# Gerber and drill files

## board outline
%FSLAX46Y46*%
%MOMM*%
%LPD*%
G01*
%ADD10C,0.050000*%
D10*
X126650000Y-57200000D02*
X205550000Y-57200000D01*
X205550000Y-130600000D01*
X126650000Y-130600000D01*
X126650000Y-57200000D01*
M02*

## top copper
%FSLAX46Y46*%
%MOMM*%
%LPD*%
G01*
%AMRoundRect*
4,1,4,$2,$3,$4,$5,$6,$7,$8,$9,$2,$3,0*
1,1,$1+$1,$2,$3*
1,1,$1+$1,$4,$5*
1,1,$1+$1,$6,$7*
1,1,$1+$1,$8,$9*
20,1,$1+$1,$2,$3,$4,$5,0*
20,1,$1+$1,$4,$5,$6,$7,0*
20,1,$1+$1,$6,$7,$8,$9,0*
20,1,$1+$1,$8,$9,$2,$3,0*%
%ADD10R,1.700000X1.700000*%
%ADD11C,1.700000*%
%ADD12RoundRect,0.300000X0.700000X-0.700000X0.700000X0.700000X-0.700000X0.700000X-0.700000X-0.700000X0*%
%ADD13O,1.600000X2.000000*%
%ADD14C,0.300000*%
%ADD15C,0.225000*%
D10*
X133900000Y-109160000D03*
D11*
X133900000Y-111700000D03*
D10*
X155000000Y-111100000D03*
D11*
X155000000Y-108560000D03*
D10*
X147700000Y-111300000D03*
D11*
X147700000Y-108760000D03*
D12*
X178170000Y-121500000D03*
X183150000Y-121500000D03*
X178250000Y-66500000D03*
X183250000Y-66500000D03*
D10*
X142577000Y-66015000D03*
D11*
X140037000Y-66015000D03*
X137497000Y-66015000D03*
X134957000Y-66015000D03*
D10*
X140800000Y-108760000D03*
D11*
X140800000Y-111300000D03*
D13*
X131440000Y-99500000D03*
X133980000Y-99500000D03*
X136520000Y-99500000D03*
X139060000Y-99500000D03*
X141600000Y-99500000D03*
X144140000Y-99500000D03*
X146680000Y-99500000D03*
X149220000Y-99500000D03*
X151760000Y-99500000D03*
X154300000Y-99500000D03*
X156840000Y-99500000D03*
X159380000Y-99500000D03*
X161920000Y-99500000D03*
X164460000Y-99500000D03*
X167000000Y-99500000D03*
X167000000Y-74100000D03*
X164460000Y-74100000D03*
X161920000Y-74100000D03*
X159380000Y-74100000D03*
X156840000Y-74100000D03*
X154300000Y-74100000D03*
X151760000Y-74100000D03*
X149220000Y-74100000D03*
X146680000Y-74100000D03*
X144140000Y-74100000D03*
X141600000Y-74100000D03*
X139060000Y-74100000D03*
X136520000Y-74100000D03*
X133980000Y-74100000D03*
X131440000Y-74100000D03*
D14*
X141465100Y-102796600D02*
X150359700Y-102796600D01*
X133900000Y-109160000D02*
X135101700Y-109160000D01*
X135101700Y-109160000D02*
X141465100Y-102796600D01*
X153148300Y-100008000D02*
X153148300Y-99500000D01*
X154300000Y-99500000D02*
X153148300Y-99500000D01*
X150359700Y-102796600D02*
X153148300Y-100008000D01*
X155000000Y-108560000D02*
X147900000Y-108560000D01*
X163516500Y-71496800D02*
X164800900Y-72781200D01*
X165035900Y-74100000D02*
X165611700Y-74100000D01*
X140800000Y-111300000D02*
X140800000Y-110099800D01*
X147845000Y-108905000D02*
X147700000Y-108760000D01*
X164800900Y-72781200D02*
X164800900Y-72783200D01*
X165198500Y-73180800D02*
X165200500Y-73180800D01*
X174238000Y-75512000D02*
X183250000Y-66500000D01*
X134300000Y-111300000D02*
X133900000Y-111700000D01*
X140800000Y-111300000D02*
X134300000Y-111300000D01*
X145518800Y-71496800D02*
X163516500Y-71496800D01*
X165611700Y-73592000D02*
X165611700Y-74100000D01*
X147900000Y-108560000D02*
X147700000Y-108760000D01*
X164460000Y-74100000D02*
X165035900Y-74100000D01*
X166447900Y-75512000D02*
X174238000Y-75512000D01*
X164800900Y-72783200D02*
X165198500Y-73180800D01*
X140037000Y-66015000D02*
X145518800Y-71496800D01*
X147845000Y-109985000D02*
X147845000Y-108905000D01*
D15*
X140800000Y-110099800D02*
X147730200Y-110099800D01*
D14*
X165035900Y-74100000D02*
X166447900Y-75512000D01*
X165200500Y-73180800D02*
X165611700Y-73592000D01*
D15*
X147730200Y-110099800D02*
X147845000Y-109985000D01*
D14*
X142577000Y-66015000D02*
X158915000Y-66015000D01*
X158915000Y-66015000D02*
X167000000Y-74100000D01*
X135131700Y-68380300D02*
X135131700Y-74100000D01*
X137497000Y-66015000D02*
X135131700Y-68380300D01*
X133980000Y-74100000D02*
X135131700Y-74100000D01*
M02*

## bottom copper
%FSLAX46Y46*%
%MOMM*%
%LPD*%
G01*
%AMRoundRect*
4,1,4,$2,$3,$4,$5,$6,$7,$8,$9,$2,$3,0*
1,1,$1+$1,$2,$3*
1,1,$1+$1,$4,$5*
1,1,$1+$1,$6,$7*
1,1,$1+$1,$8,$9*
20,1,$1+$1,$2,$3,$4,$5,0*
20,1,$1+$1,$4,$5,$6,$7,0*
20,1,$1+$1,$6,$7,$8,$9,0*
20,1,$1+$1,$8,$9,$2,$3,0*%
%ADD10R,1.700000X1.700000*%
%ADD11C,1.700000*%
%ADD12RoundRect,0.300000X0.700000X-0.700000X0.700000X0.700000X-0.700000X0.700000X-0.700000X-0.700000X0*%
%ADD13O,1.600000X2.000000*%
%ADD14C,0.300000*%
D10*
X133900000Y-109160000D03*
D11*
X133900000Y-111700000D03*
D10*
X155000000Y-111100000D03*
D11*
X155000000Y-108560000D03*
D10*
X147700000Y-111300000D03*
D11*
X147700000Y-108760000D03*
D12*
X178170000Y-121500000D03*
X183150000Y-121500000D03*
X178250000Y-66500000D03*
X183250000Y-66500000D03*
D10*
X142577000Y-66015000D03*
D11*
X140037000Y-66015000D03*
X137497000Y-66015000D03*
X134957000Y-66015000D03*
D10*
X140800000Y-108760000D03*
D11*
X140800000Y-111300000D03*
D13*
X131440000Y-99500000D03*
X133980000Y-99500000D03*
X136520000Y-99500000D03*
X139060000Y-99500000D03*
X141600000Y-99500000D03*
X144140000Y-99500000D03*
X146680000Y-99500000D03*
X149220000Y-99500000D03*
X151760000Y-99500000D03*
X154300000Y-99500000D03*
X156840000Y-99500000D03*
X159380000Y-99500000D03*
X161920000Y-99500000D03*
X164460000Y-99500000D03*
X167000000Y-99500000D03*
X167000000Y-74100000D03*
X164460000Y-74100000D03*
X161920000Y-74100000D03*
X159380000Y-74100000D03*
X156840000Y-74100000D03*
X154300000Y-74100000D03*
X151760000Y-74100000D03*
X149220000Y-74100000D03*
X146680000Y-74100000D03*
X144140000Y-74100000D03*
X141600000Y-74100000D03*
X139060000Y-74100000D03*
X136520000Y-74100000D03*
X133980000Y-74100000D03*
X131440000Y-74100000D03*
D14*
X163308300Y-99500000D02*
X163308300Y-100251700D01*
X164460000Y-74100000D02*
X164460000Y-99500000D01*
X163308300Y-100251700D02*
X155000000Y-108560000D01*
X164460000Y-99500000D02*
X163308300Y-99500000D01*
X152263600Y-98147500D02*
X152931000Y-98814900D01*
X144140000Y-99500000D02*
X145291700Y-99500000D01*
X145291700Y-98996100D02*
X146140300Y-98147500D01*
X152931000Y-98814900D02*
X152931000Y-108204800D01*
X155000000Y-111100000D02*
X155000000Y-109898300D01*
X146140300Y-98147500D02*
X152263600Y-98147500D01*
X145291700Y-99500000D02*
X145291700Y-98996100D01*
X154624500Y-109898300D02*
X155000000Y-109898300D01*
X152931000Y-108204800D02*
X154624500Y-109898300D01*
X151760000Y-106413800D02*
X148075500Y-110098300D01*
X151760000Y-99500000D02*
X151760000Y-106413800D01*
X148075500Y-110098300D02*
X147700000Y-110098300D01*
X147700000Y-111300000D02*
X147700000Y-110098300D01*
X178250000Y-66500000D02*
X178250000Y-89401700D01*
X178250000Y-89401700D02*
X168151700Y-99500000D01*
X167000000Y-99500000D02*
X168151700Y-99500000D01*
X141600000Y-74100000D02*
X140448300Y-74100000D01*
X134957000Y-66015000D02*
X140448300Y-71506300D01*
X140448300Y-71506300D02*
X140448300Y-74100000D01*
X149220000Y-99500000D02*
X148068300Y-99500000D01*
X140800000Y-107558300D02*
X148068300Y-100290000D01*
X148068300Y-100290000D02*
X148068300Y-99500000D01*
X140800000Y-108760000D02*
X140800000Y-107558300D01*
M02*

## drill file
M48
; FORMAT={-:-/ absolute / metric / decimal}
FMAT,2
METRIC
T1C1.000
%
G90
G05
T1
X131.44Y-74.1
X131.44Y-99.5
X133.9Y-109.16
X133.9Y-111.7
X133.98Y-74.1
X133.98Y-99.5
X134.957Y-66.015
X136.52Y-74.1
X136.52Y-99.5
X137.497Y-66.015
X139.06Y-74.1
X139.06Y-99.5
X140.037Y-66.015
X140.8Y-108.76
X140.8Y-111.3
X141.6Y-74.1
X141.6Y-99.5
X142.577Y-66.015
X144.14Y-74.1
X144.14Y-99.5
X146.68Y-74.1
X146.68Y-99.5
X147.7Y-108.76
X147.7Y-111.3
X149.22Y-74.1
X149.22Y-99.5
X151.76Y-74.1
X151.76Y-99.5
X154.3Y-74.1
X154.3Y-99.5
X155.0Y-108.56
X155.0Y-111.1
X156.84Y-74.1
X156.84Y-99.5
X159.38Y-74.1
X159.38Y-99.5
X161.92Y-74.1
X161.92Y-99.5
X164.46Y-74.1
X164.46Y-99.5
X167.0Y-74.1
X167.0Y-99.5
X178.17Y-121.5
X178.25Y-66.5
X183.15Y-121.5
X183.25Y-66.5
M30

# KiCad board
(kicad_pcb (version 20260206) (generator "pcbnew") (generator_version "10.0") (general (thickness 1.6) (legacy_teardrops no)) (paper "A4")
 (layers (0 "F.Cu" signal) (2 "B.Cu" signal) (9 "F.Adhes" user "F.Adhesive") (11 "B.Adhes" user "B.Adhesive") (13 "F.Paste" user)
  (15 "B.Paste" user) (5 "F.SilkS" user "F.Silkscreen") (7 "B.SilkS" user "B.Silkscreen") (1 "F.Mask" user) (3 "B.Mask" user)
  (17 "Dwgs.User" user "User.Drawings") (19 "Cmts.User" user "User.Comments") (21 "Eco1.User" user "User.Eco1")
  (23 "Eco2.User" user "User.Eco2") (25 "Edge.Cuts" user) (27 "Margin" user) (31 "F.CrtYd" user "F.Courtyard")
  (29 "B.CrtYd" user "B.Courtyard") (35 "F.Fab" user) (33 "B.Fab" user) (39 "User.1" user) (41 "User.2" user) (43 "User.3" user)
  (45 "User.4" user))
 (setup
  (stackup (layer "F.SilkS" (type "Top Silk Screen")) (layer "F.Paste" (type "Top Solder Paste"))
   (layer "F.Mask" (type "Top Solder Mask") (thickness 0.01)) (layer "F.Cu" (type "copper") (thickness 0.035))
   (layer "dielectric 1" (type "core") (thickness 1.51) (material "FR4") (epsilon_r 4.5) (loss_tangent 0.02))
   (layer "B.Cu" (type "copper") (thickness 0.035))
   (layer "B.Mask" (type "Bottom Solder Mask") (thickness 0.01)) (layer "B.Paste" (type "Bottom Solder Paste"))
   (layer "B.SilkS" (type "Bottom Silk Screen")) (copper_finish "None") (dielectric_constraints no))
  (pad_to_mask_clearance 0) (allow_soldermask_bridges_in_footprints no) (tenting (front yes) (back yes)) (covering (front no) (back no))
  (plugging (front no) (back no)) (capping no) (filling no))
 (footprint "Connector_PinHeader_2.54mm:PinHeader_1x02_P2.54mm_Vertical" (layer "F.Cu") (at 133.9 109.16)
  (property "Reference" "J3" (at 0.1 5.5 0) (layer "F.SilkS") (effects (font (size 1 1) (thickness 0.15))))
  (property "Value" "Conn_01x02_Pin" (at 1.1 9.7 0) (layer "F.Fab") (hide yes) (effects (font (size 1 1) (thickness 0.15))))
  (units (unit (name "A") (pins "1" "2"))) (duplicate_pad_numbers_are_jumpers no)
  (pad "1" thru_hole rect (at 0 0) (size 1.7 1.7) (drill 1) (layers "*.Cu" "*.Mask") (remove_unused_layers no) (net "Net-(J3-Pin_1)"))
  (pad "2" thru_hole circle (at 0 2.54) (size 1.7 1.7) (drill 1) (layers "*.Cu" "*.Mask") (remove_unused_layers no) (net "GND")))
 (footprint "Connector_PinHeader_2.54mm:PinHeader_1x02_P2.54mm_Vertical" (layer "F.Cu") (at 155 111.1 180)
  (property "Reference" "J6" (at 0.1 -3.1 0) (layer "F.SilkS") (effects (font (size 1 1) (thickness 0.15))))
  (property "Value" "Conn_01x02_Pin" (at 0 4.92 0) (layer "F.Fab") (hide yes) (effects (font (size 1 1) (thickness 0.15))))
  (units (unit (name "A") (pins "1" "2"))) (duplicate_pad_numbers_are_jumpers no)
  (pad "1" thru_hole rect (at 0 0 180) (size 1.7 1.7) (drill 1) (layers "*.Cu" "*.Mask") (remove_unused_layers no) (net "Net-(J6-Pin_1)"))
  (pad "2" thru_hole circle (at 0 2.54 180) (size 1.7 1.7) (drill 1) (layers "*.Cu" "*.Mask") (remove_unused_layers no) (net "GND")))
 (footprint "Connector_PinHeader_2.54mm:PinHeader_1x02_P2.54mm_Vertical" (layer "F.Cu") (at 147.7 111.3 180)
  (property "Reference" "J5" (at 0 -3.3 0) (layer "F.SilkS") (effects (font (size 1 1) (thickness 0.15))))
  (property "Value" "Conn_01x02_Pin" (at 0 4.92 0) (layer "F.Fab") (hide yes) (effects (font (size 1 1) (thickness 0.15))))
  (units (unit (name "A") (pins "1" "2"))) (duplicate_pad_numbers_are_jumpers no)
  (pad "1" thru_hole rect (at 0 0 180) (size 1.7 1.7) (drill 1) (layers "*.Cu" "*.Mask") (remove_unused_layers no) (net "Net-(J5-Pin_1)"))
  (pad "2" thru_hole circle (at 0 2.54 180) (size 1.7 1.7) (drill 1) (layers "*.Cu" "*.Mask") (remove_unused_layers no) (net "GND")))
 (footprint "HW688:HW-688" (layer "F.Cu") (at 186.95 94.5)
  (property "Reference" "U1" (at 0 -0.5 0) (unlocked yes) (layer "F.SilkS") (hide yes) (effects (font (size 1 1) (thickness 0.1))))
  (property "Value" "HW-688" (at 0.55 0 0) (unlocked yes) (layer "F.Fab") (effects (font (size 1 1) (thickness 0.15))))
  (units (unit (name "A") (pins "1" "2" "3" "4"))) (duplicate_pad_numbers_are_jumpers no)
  (pad "1" thru_hole roundrect (at -8.78 27 90) (size 2 2) (drill 1) (layers "*.Cu" "*.Mask") (remove_unused_layers no)
   (roundrect_rratio 0.15) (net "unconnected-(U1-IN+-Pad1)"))
  (pad "2" thru_hole roundrect (at -3.8 27 90) (size 2 2) (drill 1) (layers "*.Cu" "*.Mask") (remove_unused_layers no)
   (roundrect_rratio 0.15) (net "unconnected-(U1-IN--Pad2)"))
  (pad "3" thru_hole roundrect (at -8.7 -28 90) (size 2 2) (drill 1) (layers "*.Cu" "*.Mask") (remove_unused_layers no)
   (roundrect_rratio 0.15) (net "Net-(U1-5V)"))
  (pad "4" thru_hole roundrect (at -3.7 -28 90) (size 2 2) (drill 1) (layers "*.Cu" "*.Mask") (remove_unused_layers no)
   (roundrect_rratio 0.15) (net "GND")))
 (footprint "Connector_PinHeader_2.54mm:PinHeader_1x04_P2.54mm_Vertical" (layer "F.Cu") (at 142.577 66.015 -90)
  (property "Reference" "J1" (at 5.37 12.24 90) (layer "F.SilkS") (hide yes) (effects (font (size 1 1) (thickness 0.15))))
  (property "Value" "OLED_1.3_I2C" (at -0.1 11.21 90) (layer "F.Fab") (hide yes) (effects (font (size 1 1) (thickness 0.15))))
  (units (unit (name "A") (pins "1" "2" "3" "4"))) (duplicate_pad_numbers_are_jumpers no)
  (pad "1" thru_hole rect (at 0 0 270) (size 1.7 1.7) (drill 1) (layers "*.Cu" "*.Mask") (remove_unused_layers no) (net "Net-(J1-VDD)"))
  (pad "2" thru_hole circle (at 0 2.54 270) (size 1.7 1.7) (drill 1) (layers "*.Cu" "*.Mask") (remove_unused_layers no) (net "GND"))
  (pad "3" thru_hole circle (at 0 5.08 270) (size 1.7 1.7) (drill 1) (layers "*.Cu" "*.Mask") (remove_unused_layers no) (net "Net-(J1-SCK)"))
  (pad "4" thru_hole circle (at 0 7.62 270) (size 1.7 1.7) (drill 1) (layers "*.Cu" "*.Mask") (remove_unused_layers no) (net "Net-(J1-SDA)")))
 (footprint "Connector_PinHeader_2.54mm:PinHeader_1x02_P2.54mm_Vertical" (layer "F.Cu") (at 140.8 108.76)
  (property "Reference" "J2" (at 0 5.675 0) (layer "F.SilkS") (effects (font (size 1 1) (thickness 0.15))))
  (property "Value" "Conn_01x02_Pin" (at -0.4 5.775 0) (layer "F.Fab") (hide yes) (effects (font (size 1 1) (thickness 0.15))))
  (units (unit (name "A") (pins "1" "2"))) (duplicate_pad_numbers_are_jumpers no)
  (pad "1" thru_hole rect (at 0 0) (size 1.7 1.7) (drill 1) (layers "*.Cu" "*.Mask") (remove_unused_layers no) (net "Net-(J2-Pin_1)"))
  (pad "2" thru_hole circle (at 0 2.54) (size 1.7 1.7) (drill 1) (layers "*.Cu" "*.Mask") (remove_unused_layers no) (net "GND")))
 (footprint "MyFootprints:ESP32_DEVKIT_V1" (layer "F.Cu") (at 149.22 88.07)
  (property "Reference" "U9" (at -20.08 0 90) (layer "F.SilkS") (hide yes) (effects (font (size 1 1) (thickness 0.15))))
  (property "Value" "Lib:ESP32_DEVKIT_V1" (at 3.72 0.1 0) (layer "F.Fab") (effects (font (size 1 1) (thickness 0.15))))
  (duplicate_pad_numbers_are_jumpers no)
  (pad "1" thru_hole oval (at -17.78 11.43) (size 1.6 2) (drill 1) (layers "*.Cu" "*.Mask") (remove_unused_layers no)
   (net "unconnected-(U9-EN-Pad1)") (thermal_bridge_angle 45))
  (pad "2" thru_hole oval (at -15.24 11.43) (size 1.6 2) (drill 1) (layers "*.Cu" "*.Mask") (remove_unused_layers no)
   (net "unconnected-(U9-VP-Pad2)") (thermal_bridge_angle 45))
  (pad "3" thru_hole oval (at -12.7 11.43) (size 1.6 2) (drill 1) (layers "*.Cu" "*.Mask") (remove_unused_layers no)
   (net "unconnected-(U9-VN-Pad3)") (thermal_bridge_angle 45))
  (pad "4" thru_hole oval (at -10.16 11.43) (size 1.6 2) (drill 1) (layers "*.Cu" "*.Mask") (remove_unused_layers no)
   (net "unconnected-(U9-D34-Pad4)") (thermal_bridge_angle 45))
  (pad "5" thru_hole oval (at -7.62 11.43) (size 1.6 2) (drill 1) (layers "*.Cu" "*.Mask") (remove_unused_layers no)
   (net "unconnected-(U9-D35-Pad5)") (thermal_bridge_angle 45))
  (pad "6" thru_hole oval (at -5.08 11.43) (size 1.6 2) (drill 1) (layers "*.Cu" "*.Mask") (remove_unused_layers no) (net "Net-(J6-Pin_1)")
   (thermal_bridge_angle 45))
  (pad "7" thru_hole oval (at -2.54 11.43) (size 1.6 2) (drill 1) (layers "*.Cu" "*.Mask") (remove_unused_layers no)
   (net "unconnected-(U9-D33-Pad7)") (thermal_bridge_angle 45))
  (pad "8" thru_hole oval (at 0 11.43) (size 1.6 2) (drill 1) (layers "*.Cu" "*.Mask") (remove_unused_layers no) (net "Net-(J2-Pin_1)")
   (thermal_bridge_angle 45))
  (pad "9" thru_hole oval (at 2.54 11.43) (size 1.6 2) (drill 1) (layers "*.Cu" "*.Mask") (remove_unused_layers no) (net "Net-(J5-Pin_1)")
   (thermal_bridge_angle 45))
  (pad "10" thru_hole oval (at 5.08 11.43) (size 1.6 2) (drill 1) (layers "*.Cu" "*.Mask") (remove_unused_layers no) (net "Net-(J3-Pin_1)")
   (thermal_bridge_angle 45))
  (pad "11" thru_hole oval (at 7.62 11.43) (size 1.6 2) (drill 1) (layers "*.Cu" "*.Mask") (remove_unused_layers no)
   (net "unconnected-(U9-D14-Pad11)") (thermal_bridge_angle 45))
  (pad "12" thru_hole oval (at 10.16 11.43) (size 1.6 2) (drill 1) (layers "*.Cu" "*.Mask") (remove_unused_layers no)
   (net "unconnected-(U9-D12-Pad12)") (thermal_bridge_angle 45))
  (pad "13" thru_hole oval (at 12.7 11.43) (size 1.6 2) (drill 1) (layers "*.Cu" "*.Mask") (remove_unused_layers no)
   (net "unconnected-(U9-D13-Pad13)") (thermal_bridge_angle 45))
  (pad "14" thru_hole oval (at 15.24 11.43) (size 1.6 2) (drill 1) (layers "*.Cu" "*.Mask") (remove_unused_layers no) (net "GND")
   (thermal_bridge_angle 45))
  (pad "15" thru_hole oval (at 17.78 11.43) (size 1.6 2) (drill 1) (layers "*.Cu" "*.Mask") (remove_unused_layers no) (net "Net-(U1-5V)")
   (thermal_bridge_angle 45))
  (pad "16" thru_hole oval (at 17.78 -13.97) (size 1.6 2) (drill 1) (layers "*.Cu" "*.Mask") (remove_unused_layers no) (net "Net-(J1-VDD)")
   (thermal_bridge_angle 45))
  (pad "17" thru_hole oval (at 15.24 -13.97) (size 1.6 2) (drill 1) (layers "*.Cu" "*.Mask") (remove_unused_layers no) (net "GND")
   (thermal_bridge_angle 45))
  (pad "18" thru_hole oval (at 12.7 -13.97) (size 1.6 2) (drill 1) (layers "*.Cu" "*.Mask") (remove_unused_layers no)
   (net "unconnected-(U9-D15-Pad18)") (thermal_bridge_angle 45))
  (pad "19" thru_hole oval (at 10.16 -13.97) (size 1.6 2) (drill 1) (layers "*.Cu" "*.Mask") (remove_unused_layers no)
   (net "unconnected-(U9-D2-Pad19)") (thermal_bridge_angle 45))
  (pad "20" thru_hole oval (at 7.62 -13.97) (size 1.6 2) (drill 1) (layers "*.Cu" "*.Mask") (remove_unused_layers no)
   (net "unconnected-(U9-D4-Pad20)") (thermal_bridge_angle 45))
  (pad "21" thru_hole oval (at 5.08 -13.97) (size 1.6 2) (drill 1) (layers "*.Cu" "*.Mask") (remove_unused_layers no)
   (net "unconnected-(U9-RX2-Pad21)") (thermal_bridge_angle 45))
  (pad "22" thru_hole oval (at 2.54 -13.97) (size 1.6 2) (drill 1) (layers "*.Cu" "*.Mask") (remove_unused_layers no)
   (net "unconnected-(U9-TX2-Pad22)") (thermal_bridge_angle 45))
  (pad "23" thru_hole oval (at 0 -13.97) (size 1.6 2) (drill 1) (layers "*.Cu" "*.Mask") (remove_unused_layers no)
   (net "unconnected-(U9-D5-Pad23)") (thermal_bridge_angle 45))
  (pad "24" thru_hole oval (at -2.54 -13.97) (size 1.6 2) (drill 1) (layers "*.Cu" "*.Mask") (remove_unused_layers no)
   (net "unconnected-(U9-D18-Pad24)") (thermal_bridge_angle 45))
  (pad "25" thru_hole oval (at -5.08 -13.97) (size 1.6 2) (drill 1) (layers "*.Cu" "*.Mask") (remove_unused_layers no)
   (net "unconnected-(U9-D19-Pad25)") (thermal_bridge_angle 45))
  (pad "26" thru_hole oval (at -7.62 -13.97) (size 1.6 2) (drill 1) (layers "*.Cu" "*.Mask") (remove_unused_layers no) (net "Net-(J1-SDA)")
   (thermal_bridge_angle 45))
  (pad "27" thru_hole oval (at -10.16 -13.97) (size 1.6 2) (drill 1) (layers "*.Cu" "*.Mask") (remove_unused_layers no)
   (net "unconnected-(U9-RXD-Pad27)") (thermal_bridge_angle 45))
  (pad "28" thru_hole oval (at -12.7 -13.97) (size 1.6 2) (drill 1) (layers "*.Cu" "*.Mask") (remove_unused_layers no)
   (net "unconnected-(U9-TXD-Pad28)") (thermal_bridge_angle 45))
  (pad "29" thru_hole oval (at -15.24 -13.97) (size 1.6 2) (drill 1) (layers "*.Cu" "*.Mask") (remove_unused_layers no) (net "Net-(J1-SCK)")
   (thermal_bridge_angle 45))
  (pad "30" thru_hole oval (at -17.78 -13.97) (size 1.6 2) (drill 1) (layers "*.Cu" "*.Mask") (remove_unused_layers no)
   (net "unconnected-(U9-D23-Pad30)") (thermal_bridge_angle 45)))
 (gr_rect (start 126.65 57.2) (end 205.55 130.6) (stroke (width 0.05) (type default)) (fill no) (layer "Edge.Cuts"))
 (segment (start 141.4651 102.7966) (end 150.3597 102.7966) (width 0.3) (layer "F.Cu") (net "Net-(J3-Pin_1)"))
 (segment (start 133.9 109.16) (end 135.1017 109.16) (width 0.3) (layer "F.Cu") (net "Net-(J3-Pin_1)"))
 (segment (start 135.1017 109.16) (end 141.4651 102.7966) (width 0.3) (layer "F.Cu") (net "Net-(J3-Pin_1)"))
 (segment (start 153.1483 100.008) (end 153.1483 99.5) (width 0.3) (layer "F.Cu") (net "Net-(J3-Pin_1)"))
 (segment (start 154.3 99.5) (end 153.1483 99.5) (width 0.3) (layer "F.Cu") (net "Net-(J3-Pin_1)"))
 (segment (start 150.3597 102.7966) (end 153.1483 100.008) (width 0.3) (layer "F.Cu") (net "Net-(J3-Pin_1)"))
 (segment (start 155 108.56) (end 147.9 108.56) (width 0.3) (layer "F.Cu") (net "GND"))
 (segment (start 163.5165 71.4968) (end 164.8009 72.7812) (width 0.3) (layer "F.Cu") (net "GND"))
 (segment (start 165.0359 74.1) (end 165.6117 74.1) (width 0.3) (layer "F.Cu") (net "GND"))
 (segment (start 140.8 111.3) (end 140.8 110.0998) (width 0.3) (layer "F.Cu") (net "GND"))
 (segment (start 147.845 108.905) (end 147.7 108.76) (width 0.3) (layer "F.Cu") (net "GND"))
 (segment (start 164.8009 72.7812) (end 164.8009 72.7832) (width 0.3) (layer "F.Cu") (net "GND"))
 (segment (start 165.1985 73.1808) (end 165.2005 73.1808) (width 0.3) (layer "F.Cu") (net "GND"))
 (segment (start 174.238 75.512) (end 183.25 66.5) (width 0.3) (layer "F.Cu") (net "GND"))
 (segment (start 134.3 111.3) (end 133.9 111.7) (width 0.3) (layer "F.Cu") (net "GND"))
 (segment (start 140.8 111.3) (end 134.3 111.3) (width 0.3) (layer "F.Cu") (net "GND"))
 (segment (start 145.5188 71.4968) (end 163.5165 71.4968) (width 0.3) (layer "F.Cu") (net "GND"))
 (segment (start 165.6117 73.592) (end 165.6117 74.1) (width 0.3) (layer "F.Cu") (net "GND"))
 (segment (start 147.9 108.56) (end 147.7 108.76) (width 0.3) (layer "F.Cu") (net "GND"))
 (segment (start 164.46 74.1) (end 165.0359 74.1) (width 0.3) (layer "F.Cu") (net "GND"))
 (segment (start 166.4479 75.512) (end 174.238 75.512) (width 0.3) (layer "F.Cu") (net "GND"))
 (segment (start 164.8009 72.7832) (end 165.1985 73.1808) (width 0.3) (layer "F.Cu") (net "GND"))
 (segment (start 140.037 66.015) (end 145.5188 71.4968) (width 0.3) (layer "F.Cu") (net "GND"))
 (segment (start 147.845 109.985) (end 147.845 108.905) (width 0.3) (layer "F.Cu") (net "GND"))
 (segment (start 140.8 110.0998) (end 147.7302 110.0998) (width 0.225) (layer "F.Cu") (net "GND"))
 (segment (start 165.0359 74.1) (end 166.4479 75.512) (width 0.3) (layer "F.Cu") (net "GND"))
 (segment (start 165.2005 73.1808) (end 165.6117 73.592) (width 0.3) (layer "F.Cu") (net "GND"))
 (segment (start 147.7302 110.0998) (end 147.845 109.985) (width 0.225) (layer "F.Cu") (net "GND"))
 (segment (start 163.3083 99.5) (end 163.3083 100.2517) (width 0.3) (layer "B.Cu") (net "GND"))
 (segment (start 164.46 74.1) (end 164.46 99.5) (width 0.3) (layer "B.Cu") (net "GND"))
 (segment (start 163.3083 100.2517) (end 155 108.56) (width 0.3) (layer "B.Cu") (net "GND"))
 (segment (start 164.46 99.5) (end 163.3083 99.5) (width 0.3) (layer "B.Cu") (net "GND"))
 (segment (start 152.2636 98.1475) (end 152.931 98.8149) (width 0.3) (layer "B.Cu") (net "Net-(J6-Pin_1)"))
 (segment (start 144.14 99.5) (end 145.2917 99.5) (width 0.3) (layer "B.Cu") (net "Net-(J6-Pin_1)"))
 (segment (start 145.2917 98.9961) (end 146.1403 98.1475) (width 0.3) (layer "B.Cu") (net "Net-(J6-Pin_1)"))
 (segment (start 152.931 98.8149) (end 152.931 108.2048) (width 0.3) (layer "B.Cu") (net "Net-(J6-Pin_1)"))
 (segment (start 155 111.1) (end 155 109.8983) (width 0.3) (layer "B.Cu") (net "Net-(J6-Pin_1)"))
 (segment (start 146.1403 98.1475) (end 152.2636 98.1475) (width 0.3) (layer "B.Cu") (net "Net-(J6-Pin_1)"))
 (segment (start 145.2917 99.5) (end 145.2917 98.9961) (width 0.3) (layer "B.Cu") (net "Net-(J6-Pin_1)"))
 (segment (start 154.6245 109.8983) (end 155 109.8983) (width 0.3) (layer "B.Cu") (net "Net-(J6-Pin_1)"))
 (segment (start 152.931 108.2048) (end 154.6245 109.8983) (width 0.3) (layer "B.Cu") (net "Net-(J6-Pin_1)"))
 (segment (start 151.76 106.4138) (end 148.0755 110.0983) (width 0.3) (layer "B.Cu") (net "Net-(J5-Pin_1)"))
 (segment (start 151.76 99.5) (end 151.76 106.4138) (width 0.3) (layer "B.Cu") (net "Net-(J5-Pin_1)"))
 (segment (start 148.0755 110.0983) (end 147.7 110.0983) (width 0.3) (layer "B.Cu") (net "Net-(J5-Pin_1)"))
 (segment (start 147.7 111.3) (end 147.7 110.0983) (width 0.3) (layer "B.Cu") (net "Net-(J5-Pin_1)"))
 (segment (start 178.25 66.5) (end 178.25 89.4017) (width 0.3) (layer "B.Cu") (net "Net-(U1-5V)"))
 (segment (start 178.25 89.4017) (end 168.1517 99.5) (width 0.3) (layer "B.Cu") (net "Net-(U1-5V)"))
 (segment (start 167 99.5) (end 168.1517 99.5) (width 0.3) (layer "B.Cu") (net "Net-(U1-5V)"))
 (segment (start 142.577 66.015) (end 158.915 66.015) (width 0.3) (layer "F.Cu") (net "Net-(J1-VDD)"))
 (segment (start 158.915 66.015) (end 167 74.1) (width 0.3) (layer "F.Cu") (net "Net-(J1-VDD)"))
 (segment (start 135.1317 68.3803) (end 135.1317 74.1) (width 0.3) (layer "F.Cu") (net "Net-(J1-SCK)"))
 (segment (start 137.497 66.015) (end 135.1317 68.3803) (width 0.3) (layer "F.Cu") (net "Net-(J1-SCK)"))
 (segment (start 133.98 74.1) (end 135.1317 74.1) (width 0.3) (layer "F.Cu") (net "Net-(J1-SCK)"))
 (segment (start 141.6 74.1) (end 140.4483 74.1) (width 0.3) (layer "B.Cu") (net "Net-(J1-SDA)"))
 (segment (start 134.957 66.015) (end 140.4483 71.5063) (width 0.3) (layer "B.Cu") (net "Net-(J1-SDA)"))
 (segment (start 140.4483 71.5063) (end 140.4483 74.1) (width 0.3) (layer "B.Cu") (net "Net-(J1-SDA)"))
 (segment (start 149.22 99.5) (end 148.0683 99.5) (width 0.3) (layer "B.Cu") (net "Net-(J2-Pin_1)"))
 (segment (start 140.8 107.5583) (end 148.0683 100.29) (width 0.3) (layer "B.Cu") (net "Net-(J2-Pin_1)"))
 (segment (start 148.0683 100.29) (end 148.0683 99.5) (width 0.3) (layer "B.Cu") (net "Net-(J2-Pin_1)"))
 (segment (start 140.8 108.76) (end 140.8 107.5583) (width 0.3) (layer "B.Cu") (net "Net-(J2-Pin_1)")))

